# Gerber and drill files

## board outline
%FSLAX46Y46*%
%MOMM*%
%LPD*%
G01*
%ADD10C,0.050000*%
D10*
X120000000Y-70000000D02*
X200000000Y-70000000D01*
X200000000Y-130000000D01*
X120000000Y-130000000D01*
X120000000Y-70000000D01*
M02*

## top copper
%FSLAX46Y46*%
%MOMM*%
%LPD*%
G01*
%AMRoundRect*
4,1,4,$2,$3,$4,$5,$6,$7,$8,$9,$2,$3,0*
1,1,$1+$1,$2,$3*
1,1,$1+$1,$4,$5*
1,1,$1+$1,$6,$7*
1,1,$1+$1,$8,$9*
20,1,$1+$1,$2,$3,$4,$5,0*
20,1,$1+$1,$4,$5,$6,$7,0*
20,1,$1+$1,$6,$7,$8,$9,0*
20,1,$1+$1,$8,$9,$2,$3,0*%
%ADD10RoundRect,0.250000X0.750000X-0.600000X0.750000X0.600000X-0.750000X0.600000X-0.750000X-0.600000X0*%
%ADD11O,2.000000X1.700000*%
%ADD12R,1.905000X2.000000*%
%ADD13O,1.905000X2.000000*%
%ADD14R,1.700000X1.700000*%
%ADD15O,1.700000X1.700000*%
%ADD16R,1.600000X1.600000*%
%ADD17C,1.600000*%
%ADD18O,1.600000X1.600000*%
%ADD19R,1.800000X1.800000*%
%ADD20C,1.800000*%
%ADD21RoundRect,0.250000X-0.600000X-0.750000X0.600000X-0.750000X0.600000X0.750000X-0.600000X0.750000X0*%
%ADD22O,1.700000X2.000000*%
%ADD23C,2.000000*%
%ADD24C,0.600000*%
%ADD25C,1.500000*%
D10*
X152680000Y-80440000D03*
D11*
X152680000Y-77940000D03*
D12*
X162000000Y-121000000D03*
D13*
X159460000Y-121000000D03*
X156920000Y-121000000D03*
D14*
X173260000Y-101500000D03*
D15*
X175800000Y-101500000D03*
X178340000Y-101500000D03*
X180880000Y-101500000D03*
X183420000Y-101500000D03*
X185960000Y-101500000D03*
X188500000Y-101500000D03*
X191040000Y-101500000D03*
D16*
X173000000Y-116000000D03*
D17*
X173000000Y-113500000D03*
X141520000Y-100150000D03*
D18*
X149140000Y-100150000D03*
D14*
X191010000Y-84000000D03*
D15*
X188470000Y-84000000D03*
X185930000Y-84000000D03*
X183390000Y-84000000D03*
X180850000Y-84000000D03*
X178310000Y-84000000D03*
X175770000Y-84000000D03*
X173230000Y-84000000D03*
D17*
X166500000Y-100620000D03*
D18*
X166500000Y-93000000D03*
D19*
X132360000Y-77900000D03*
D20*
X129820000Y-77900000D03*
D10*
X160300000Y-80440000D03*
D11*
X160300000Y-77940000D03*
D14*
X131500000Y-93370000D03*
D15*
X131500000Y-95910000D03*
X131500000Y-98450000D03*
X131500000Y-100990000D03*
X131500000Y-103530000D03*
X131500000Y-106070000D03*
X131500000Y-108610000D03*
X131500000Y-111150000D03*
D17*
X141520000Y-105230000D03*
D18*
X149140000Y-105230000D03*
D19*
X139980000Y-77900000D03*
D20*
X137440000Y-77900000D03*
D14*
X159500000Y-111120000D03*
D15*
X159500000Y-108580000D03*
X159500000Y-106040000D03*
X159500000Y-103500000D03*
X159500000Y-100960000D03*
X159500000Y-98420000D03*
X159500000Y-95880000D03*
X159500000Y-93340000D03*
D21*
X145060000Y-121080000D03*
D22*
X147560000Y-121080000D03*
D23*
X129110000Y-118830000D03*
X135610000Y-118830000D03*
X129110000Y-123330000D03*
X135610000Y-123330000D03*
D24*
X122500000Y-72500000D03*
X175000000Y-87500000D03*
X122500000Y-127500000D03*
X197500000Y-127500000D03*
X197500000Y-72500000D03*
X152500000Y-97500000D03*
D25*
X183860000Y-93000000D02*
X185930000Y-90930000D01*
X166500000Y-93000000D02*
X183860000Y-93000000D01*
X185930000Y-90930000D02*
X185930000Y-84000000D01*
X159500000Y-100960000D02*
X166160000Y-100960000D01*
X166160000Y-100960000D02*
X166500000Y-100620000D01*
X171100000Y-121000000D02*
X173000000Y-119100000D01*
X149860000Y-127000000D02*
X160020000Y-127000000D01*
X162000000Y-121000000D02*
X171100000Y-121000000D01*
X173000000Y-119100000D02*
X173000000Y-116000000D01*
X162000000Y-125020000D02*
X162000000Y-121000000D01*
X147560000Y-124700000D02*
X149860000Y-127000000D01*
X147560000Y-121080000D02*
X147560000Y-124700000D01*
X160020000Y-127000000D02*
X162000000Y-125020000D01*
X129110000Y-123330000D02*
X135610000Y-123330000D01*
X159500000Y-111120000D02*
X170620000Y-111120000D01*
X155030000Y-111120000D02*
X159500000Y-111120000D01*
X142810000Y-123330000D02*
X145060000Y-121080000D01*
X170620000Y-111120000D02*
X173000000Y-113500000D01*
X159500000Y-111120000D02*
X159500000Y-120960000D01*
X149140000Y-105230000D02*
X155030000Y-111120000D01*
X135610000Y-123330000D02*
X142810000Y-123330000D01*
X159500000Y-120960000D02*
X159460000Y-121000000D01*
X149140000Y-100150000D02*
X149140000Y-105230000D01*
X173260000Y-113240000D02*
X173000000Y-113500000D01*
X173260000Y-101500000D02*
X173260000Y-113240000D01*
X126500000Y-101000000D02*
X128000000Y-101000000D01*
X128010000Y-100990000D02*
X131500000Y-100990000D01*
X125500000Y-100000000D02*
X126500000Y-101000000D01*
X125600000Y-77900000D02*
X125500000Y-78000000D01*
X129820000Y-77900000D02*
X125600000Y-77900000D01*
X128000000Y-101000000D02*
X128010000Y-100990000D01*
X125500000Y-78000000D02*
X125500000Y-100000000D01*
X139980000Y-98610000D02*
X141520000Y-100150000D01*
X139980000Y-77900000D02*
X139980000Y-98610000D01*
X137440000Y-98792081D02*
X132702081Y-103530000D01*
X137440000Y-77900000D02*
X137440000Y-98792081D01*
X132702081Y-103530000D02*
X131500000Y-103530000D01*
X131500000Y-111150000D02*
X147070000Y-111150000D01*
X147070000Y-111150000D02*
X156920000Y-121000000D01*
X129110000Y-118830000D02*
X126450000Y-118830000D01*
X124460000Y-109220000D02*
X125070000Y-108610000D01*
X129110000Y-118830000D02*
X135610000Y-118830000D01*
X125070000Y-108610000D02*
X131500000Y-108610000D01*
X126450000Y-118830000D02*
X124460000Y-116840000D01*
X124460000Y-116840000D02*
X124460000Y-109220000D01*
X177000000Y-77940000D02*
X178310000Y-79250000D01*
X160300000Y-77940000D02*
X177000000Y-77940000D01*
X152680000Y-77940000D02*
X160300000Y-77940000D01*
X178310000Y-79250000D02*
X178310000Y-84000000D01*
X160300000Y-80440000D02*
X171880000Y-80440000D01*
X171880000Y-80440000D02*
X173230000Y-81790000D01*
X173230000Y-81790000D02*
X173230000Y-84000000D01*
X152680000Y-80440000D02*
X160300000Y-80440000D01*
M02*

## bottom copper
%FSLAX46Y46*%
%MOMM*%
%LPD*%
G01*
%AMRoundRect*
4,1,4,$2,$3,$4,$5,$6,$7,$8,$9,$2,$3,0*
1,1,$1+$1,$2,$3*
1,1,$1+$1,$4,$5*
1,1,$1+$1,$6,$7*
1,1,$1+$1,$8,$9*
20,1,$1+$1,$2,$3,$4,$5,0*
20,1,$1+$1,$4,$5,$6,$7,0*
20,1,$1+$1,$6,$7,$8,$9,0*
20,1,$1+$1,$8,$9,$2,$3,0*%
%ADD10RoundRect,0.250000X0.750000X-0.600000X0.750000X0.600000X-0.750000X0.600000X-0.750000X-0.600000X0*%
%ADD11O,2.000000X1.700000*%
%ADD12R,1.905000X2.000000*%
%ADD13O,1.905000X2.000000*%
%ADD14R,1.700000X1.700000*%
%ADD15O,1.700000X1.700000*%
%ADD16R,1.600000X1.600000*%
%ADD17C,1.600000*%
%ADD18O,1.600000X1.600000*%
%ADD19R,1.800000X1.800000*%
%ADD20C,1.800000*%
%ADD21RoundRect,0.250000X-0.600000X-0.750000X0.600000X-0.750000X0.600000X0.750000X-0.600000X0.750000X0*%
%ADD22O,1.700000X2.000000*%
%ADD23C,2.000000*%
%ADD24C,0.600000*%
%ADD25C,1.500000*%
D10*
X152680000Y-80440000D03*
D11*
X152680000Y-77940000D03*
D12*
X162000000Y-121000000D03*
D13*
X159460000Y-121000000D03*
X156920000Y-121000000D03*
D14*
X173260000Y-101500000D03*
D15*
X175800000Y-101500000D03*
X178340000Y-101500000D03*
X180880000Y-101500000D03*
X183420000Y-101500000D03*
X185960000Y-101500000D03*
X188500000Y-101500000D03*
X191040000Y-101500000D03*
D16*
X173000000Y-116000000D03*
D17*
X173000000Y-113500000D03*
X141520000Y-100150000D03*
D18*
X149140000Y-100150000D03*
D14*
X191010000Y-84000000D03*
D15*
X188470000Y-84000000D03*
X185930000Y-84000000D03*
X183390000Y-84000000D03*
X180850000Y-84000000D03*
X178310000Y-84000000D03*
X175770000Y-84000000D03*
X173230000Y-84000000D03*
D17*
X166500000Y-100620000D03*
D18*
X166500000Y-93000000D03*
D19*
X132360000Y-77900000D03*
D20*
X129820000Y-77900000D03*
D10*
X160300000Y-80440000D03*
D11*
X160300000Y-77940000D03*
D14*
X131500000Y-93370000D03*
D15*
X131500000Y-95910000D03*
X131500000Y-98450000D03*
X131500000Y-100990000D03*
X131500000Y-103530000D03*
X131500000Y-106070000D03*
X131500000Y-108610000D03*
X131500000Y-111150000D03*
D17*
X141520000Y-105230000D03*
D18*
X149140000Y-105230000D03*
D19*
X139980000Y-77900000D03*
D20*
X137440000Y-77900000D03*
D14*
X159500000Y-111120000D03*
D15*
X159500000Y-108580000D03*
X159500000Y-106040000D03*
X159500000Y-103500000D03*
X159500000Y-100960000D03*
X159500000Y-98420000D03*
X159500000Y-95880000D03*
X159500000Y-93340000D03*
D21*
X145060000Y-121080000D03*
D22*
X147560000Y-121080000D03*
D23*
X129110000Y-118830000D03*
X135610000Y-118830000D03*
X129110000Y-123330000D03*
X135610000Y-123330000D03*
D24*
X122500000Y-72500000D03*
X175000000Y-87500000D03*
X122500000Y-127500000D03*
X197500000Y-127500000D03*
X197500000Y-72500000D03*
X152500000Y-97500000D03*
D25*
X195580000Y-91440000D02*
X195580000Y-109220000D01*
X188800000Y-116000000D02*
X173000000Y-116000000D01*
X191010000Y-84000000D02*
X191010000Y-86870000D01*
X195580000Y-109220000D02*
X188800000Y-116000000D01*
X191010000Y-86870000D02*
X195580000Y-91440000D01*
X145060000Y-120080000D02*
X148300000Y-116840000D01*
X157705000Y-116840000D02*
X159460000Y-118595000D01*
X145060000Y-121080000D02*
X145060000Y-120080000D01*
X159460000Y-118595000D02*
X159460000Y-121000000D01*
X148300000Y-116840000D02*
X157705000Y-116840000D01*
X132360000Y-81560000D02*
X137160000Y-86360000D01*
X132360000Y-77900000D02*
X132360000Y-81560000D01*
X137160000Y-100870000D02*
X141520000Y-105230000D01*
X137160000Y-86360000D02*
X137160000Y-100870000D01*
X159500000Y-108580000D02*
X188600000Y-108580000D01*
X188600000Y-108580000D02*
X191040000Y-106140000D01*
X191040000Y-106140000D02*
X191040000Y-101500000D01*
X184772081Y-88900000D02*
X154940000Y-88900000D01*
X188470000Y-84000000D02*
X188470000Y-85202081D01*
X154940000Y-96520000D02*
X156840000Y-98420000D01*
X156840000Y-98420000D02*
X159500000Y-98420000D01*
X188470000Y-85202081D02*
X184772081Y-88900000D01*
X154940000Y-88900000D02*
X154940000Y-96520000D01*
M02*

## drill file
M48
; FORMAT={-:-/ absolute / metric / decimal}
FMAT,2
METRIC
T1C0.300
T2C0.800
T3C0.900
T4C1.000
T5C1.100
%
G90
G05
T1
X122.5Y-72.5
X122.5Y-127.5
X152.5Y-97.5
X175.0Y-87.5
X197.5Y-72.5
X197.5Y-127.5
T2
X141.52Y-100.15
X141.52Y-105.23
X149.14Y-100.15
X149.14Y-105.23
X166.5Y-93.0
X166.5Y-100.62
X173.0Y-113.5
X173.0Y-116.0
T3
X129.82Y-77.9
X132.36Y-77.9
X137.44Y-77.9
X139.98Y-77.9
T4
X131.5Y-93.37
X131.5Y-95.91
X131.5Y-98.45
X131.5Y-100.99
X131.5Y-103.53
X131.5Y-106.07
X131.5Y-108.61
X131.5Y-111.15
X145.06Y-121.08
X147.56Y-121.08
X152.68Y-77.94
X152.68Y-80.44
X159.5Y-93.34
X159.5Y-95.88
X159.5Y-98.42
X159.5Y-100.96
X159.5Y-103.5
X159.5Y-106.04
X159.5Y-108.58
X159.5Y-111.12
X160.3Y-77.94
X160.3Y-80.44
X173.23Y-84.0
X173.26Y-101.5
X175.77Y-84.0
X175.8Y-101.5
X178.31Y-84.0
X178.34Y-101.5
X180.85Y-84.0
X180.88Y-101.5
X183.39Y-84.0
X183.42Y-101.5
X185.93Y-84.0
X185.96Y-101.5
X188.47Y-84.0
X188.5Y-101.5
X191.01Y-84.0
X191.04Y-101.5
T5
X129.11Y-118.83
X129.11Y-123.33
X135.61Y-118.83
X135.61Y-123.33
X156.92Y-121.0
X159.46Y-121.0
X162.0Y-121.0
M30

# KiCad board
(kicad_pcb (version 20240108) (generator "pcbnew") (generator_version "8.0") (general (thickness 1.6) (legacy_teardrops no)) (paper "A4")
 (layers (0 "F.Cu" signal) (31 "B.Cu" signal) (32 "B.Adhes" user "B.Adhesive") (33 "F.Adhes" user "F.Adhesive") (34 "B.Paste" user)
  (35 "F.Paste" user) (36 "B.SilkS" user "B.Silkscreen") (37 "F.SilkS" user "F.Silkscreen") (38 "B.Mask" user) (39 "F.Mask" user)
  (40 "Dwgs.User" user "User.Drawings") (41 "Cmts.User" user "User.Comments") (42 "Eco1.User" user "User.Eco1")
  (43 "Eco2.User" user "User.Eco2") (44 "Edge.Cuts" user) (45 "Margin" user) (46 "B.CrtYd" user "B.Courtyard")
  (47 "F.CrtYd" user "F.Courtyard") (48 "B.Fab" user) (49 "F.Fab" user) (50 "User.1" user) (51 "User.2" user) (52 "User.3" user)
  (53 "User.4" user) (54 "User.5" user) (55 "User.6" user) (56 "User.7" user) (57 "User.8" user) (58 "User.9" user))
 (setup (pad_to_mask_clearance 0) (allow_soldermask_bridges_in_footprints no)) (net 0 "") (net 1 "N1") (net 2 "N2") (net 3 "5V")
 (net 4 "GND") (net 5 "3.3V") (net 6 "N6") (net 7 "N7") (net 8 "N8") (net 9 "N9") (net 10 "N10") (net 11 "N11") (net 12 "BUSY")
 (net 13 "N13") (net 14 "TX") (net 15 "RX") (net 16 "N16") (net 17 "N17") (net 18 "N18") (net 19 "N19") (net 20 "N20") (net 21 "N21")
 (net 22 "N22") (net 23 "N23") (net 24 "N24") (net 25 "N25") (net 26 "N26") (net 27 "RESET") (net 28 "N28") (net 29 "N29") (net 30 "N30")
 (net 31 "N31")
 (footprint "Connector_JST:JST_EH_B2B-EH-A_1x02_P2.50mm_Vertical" (layer "F.Cu") (at 152.68 80.44 90)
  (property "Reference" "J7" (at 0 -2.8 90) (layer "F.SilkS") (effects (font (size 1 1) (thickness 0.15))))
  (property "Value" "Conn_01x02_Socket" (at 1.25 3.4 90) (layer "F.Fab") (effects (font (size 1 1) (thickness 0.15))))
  (pad "1" thru_hole roundrect (at 0 0 90) (size 1.7 2) (drill 1) (layers "*.Cu" "*.Mask") (remove_unused_layers no)
   (roundrect_rratio 0.147059) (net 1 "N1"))
  (pad "2" thru_hole oval (at 2.5 0 90) (size 1.7 2) (drill 1) (layers "*.Cu" "*.Mask") (remove_unused_layers no) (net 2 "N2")))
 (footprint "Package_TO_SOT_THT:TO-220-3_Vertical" (layer "F.Cu") (at 162 121 180)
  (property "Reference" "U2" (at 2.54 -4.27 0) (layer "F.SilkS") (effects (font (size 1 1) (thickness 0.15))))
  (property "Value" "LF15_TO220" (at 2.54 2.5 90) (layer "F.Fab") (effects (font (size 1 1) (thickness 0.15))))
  (pad "1" thru_hole rect (at 0 0 180) (size 1.905 2) (drill 1.1) (layers "*.Cu" "*.Mask") (remove_unused_layers no) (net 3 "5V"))
  (pad "2" thru_hole oval (at 2.54 0 180) (size 1.905 2) (drill 1.1) (layers "*.Cu" "*.Mask") (remove_unused_layers no) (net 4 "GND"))
  (pad "3" thru_hole oval (at 5.08 0 180) (size 1.905 2) (drill 1.1) (layers "*.Cu" "*.Mask") (remove_unused_layers no) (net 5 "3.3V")))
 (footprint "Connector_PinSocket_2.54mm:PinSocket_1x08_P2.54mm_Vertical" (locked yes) (layer "F.Cu") (at 173.26 101.5 90)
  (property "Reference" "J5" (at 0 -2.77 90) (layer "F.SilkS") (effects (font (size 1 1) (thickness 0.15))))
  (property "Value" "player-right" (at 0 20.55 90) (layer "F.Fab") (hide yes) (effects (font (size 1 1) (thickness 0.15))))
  (pad "1" thru_hole rect (at 0 0 90) (size 1.7 1.7) (drill 1) (layers "*.Cu" "*.Mask") (remove_unused_layers no) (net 4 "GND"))
  (pad "2" thru_hole oval (at 0 2.54 90) (size 1.7 1.7) (drill 1) (layers "*.Cu" "*.Mask") (remove_unused_layers no) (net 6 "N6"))
  (pad "3" thru_hole oval (at 0 5.08 90) (size 1.7 1.7) (drill 1) (layers "*.Cu" "*.Mask") (remove_unused_layers no) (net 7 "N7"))
  (pad "4" thru_hole oval (at 0 7.62 90) (size 1.7 1.7) (drill 1) (layers "*.Cu" "*.Mask") (remove_unused_layers no) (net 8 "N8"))
  (pad "5" thru_hole oval (at 0 10.16 90) (size 1.7 1.7) (drill 1) (layers "*.Cu" "*.Mask") (remove_unused_layers no) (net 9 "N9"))
  (pad "6" thru_hole oval (at 0 12.7 90) (size 1.7 1.7) (drill 1) (layers "*.Cu" "*.Mask") (remove_unused_layers no) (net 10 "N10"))
  (pad "7" thru_hole oval (at 0 15.24 90) (size 1.7 1.7) (drill 1) (layers "*.Cu" "*.Mask") (remove_unused_layers no) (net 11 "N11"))
  (pad "8" thru_hole oval (at 0 17.78 90) (size 1.7 1.7) (drill 1) (layers "*.Cu" "*.Mask") (remove_unused_layers no) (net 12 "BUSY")))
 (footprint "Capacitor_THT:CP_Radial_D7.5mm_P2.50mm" (layer "F.Cu") (at 173 116 90)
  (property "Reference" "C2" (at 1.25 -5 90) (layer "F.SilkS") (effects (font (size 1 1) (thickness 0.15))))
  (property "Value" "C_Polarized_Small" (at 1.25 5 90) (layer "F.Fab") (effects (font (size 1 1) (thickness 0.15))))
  (pad "1" thru_hole rect (at 0 0 90) (size 1.6 1.6) (drill 0.8) (layers "*.Cu" "*.Mask") (remove_unused_layers no) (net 3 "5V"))
  (pad "2" thru_hole circle (at 2.5 0 90) (size 1.6 1.6) (drill 0.8) (layers "*.Cu" "*.Mask") (remove_unused_layers no) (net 4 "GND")))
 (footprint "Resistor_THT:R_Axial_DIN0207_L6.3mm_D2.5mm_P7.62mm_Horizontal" (layer "F.Cu") (at 141.52 100.15)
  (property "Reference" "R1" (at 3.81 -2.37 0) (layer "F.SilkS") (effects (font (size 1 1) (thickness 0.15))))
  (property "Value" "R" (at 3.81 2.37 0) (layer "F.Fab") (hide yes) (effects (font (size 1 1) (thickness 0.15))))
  (pad "1" thru_hole circle (at 0 0) (size 1.6 1.6) (drill 0.8) (layers "*.Cu" "*.Mask") (remove_unused_layers no) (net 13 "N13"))
  (pad "2" thru_hole oval (at 7.62 0) (size 1.6 1.6) (drill 0.8) (layers "*.Cu" "*.Mask") (remove_unused_layers no) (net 4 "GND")))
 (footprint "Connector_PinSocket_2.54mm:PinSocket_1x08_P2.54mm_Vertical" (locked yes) (layer "F.Cu") (at 191.01 84 -90)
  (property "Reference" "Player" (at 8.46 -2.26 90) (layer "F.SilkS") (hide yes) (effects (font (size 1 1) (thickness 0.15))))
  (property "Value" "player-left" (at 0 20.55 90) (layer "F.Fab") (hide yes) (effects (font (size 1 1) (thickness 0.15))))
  (pad "1" thru_hole rect (at 0 0 270) (size 1.7 1.7) (drill 1) (layers "*.Cu" "*.Mask") (remove_unused_layers no) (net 3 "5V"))
  (pad "2" thru_hole oval (at 0 2.54 270) (size 1.7 1.7) (drill 1) (layers "*.Cu" "*.Mask") (remove_unused_layers no) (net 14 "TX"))
  (pad "3" thru_hole oval (at 0 5.08 270) (size 1.7 1.7) (drill 1) (layers "*.Cu" "*.Mask") (remove_unused_layers no) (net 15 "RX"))
  (pad "4" thru_hole oval (at 0 7.62 270) (size 1.7 1.7) (drill 1) (layers "*.Cu" "*.Mask") (remove_unused_layers no) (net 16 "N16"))
  (pad "5" thru_hole oval (at 0 10.16 270) (size 1.7 1.7) (drill 1) (layers "*.Cu" "*.Mask") (remove_unused_layers no) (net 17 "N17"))
  (pad "6" thru_hole oval (at 0 12.7 270) (size 1.7 1.7) (drill 1) (layers "*.Cu" "*.Mask") (remove_unused_layers no) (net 2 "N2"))
  (pad "7" thru_hole oval (at 0 15.24 270) (size 1.7 1.7) (drill 1) (layers "*.Cu" "*.Mask") (remove_unused_layers no) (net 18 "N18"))
  (pad "8" thru_hole oval (at 0 17.78 270) (size 1.7 1.7) (drill 1) (layers "*.Cu" "*.Mask") (remove_unused_layers no) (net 1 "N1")))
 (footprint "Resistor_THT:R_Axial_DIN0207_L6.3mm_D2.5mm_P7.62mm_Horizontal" (layer "F.Cu") (at 166.5 100.62 90)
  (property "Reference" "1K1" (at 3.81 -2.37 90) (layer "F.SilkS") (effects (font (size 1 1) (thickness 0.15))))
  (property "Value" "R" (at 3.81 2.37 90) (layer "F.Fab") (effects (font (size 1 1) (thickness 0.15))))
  (pad "1" thru_hole circle (at 0 0 90) (size 1.6 1.6) (drill 0.8) (layers "*.Cu" "*.Mask") (remove_unused_layers no) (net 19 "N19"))
  (pad "2" thru_hole oval (at 7.62 0 90) (size 1.6 1.6) (drill 0.8) (layers "*.Cu" "*.Mask") (remove_unused_layers no) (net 15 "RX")))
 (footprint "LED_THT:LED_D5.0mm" (layer "F.Cu") (at 132.36 77.9 180)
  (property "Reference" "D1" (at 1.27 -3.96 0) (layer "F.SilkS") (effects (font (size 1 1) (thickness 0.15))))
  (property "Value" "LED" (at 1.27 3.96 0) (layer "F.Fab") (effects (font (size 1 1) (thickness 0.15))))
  (pad "1" thru_hole rect (at 0 0 180) (size 1.8 1.8) (drill 0.9) (layers "*.Cu" "*.Mask") (remove_unused_layers no) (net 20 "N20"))
  (pad "2" thru_hole circle (at 2.54 0 180) (size 1.8 1.8) (drill 0.9) (layers "*.Cu" "*.Mask") (remove_unused_layers no) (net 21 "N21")))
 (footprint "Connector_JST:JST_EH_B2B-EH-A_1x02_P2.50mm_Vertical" (layer "F.Cu") (at 160.3 80.44 90)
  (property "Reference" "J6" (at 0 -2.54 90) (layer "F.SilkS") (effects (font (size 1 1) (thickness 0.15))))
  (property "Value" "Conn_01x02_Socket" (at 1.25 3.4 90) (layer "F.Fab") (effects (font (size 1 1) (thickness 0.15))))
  (pad "1" thru_hole roundrect (at 0 0 90) (size 1.7 2) (drill 1) (layers "*.Cu" "*.Mask") (remove_unused_layers no)
   (roundrect_rratio 0.147059) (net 1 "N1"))
  (pad "2" thru_hole oval (at 2.5 0 90) (size 1.7 2) (drill 1) (layers "*.Cu" "*.Mask") (remove_unused_layers no) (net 2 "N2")))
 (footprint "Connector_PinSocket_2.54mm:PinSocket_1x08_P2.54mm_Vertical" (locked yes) (layer "F.Cu") (at 131.5 93.37)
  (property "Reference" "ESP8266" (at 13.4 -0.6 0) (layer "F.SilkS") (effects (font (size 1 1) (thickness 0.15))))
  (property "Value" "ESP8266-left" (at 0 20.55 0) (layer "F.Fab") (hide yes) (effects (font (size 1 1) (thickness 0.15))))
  (pad "1" thru_hole rect (at 0 0) (size 1.7 1.7) (drill 1) (layers "*.Cu" "*.Mask") (remove_unused_layers no) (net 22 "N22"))
  (pad "2" thru_hole oval (at 0 2.54) (size 1.7 1.7) (drill 1) (layers "*.Cu" "*.Mask") (remove_unused_layers no) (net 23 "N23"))
  (pad "3" thru_hole oval (at 0 5.08) (size 1.7 1.7) (drill 1) (layers "*.Cu" "*.Mask") (remove_unused_layers no) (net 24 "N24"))
  (pad "4" thru_hole oval (at 0 7.62) (size 1.7 1.7) (drill 1) (layers "*.Cu" "*.Mask") (remove_unused_layers no) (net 21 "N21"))
  (pad "5" thru_hole oval (at 0 10.16) (size 1.7 1.7) (drill 1) (layers "*.Cu" "*.Mask") (remove_unused_layers no) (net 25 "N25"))
  (pad "6" thru_hole oval (at 0 12.7) (size 1.7 1.7) (drill 1) (layers "*.Cu" "*.Mask") (remove_unused_layers no) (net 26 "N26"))
  (pad "7" thru_hole oval (at 0 15.24) (size 1.7 1.7) (drill 1) (layers "*.Cu" "*.Mask") (remove_unused_layers no) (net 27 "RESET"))
  (pad "8" thru_hole oval (at 0 17.78) (size 1.7 1.7) (drill 1) (layers "*.Cu" "*.Mask") (remove_unused_layers no) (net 5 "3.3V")))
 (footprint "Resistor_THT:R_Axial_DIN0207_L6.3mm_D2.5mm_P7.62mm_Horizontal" (layer "F.Cu") (at 141.52 105.23)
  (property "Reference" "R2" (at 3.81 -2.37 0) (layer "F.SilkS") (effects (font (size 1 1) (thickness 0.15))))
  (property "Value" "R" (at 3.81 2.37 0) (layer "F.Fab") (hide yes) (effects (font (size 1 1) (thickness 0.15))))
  (pad "1" thru_hole circle (at 0 0) (size 1.6 1.6) (drill 0.8) (layers "*.Cu" "*.Mask") (remove_unused_layers no) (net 20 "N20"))
  (pad "2" thru_hole oval (at 7.62 0) (size 1.6 1.6) (drill 0.8) (layers "*.Cu" "*.Mask") (remove_unused_layers no) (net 4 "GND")))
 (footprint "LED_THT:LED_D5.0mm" (layer "F.Cu") (at 139.98 77.9 180)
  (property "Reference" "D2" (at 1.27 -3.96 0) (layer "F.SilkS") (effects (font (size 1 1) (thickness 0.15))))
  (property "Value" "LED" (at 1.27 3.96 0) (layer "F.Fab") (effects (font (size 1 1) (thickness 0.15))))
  (pad "1" thru_hole rect (at 0 0 180) (size 1.8 1.8) (drill 0.9) (layers "*.Cu" "*.Mask") (remove_unused_layers no) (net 13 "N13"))
  (pad "2" thru_hole circle (at 2.54 0 180) (size 1.8 1.8) (drill 0.9) (layers "*.Cu" "*.Mask") (remove_unused_layers no) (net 25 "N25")))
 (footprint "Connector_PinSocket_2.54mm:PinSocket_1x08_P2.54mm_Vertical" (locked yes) (layer "F.Cu") (at 159.5 111.12 180)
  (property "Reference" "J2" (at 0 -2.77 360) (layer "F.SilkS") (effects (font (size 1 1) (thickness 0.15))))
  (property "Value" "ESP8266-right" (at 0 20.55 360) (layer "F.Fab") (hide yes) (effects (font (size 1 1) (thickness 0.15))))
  (pad "1" thru_hole rect (at 0 0 180) (size 1.7 1.7) (drill 1) (layers "*.Cu" "*.Mask") (remove_unused_layers no) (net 4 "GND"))
  (pad "2" thru_hole oval (at 0 2.54 180) (size 1.7 1.7) (drill 1) (layers "*.Cu" "*.Mask") (remove_unused_layers no) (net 12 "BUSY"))
  (pad "3" thru_hole oval (at 0 5.08 180) (size 1.7 1.7) (drill 1) (layers "*.Cu" "*.Mask") (remove_unused_layers no) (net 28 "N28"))
  (pad "4" thru_hole oval (at 0 7.62 180) (size 1.7 1.7) (drill 1) (layers "*.Cu" "*.Mask") (remove_unused_layers no) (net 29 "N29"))
  (pad "5" thru_hole oval (at 0 10.16 180) (size 1.7 1.7) (drill 1) (layers "*.Cu" "*.Mask") (remove_unused_layers no) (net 19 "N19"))
  (pad "6" thru_hole oval (at 0 12.7 180) (size 1.7 1.7) (drill 1) (layers "*.Cu" "*.Mask") (remove_unused_layers no) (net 14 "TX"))
  (pad "7" thru_hole oval (at 0 15.24 180) (size 1.7 1.7) (drill 1) (layers "*.Cu" "*.Mask") (remove_unused_layers no) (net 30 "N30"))
  (pad "8" thru_hole oval (at 0 17.78 180) (size 1.7 1.7) (drill 1) (layers "*.Cu" "*.Mask") (remove_unused_layers no) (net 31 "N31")))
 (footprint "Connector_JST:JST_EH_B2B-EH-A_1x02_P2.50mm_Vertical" (layer "F.Cu") (at 145.06 121.08)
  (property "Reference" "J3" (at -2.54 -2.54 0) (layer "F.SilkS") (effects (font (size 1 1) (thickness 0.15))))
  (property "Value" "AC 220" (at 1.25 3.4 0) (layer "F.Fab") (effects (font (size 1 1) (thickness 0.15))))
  (pad "1" thru_hole roundrect (at 0 0) (size 1.7 2) (drill 1) (layers "*.Cu" "*.Mask") (remove_unused_layers no)
   (roundrect_rratio 0.147059) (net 4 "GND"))
  (pad "2" thru_hole oval (at 2.5 0) (size 1.7 2) (drill 1) (layers "*.Cu" "*.Mask") (remove_unused_layers no) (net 3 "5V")))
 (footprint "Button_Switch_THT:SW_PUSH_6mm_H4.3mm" (layer "F.Cu") (at 129.11 118.83)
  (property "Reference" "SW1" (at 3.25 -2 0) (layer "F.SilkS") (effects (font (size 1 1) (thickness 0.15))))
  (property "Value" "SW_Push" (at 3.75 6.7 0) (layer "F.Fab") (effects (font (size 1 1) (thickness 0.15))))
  (pad "1" thru_hole circle (at 0 0 90) (size 2 2) (drill 1.1) (layers "*.Cu" "*.Mask") (remove_unused_layers no) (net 27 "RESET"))
  (pad "1" thru_hole circle (at 6.5 0 90) (size 2 2) (drill 1.1) (layers "*.Cu" "*.Mask") (remove_unused_layers no) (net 27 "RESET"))
  (pad "2" thru_hole circle (at 0 4.5 90) (size 2 2) (drill 1.1) (layers "*.Cu" "*.Mask") (remove_unused_layers no) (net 4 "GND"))
  (pad "2" thru_hole circle (at 6.5 4.5 90) (size 2 2) (drill 1.1) (layers "*.Cu" "*.Mask") (remove_unused_layers no) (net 4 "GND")))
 (gr_rect (start 120 70) (end 200 130) (stroke (width 0.05) (type default)) (fill none) (layer "Edge.Cuts"))
 (via (at 122.5 72.5) (size 0.6) (drill 0.3) (layers "F.Cu" "B.Cu") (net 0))
 (via (at 175 87.5) (size 0.6) (drill 0.3) (layers "F.Cu" "B.Cu") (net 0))
 (via (at 122.5 127.5) (size 0.6) (drill 0.3) (layers "F.Cu" "B.Cu") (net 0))
 (via (at 197.5 127.5) (size 0.6) (drill 0.3) (layers "F.Cu" "B.Cu") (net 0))
 (via (at 197.5 72.5) (size 0.6) (drill 0.3) (layers "F.Cu" "B.Cu") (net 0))
 (via (at 152.5 97.5) (size 0.6) (drill 0.3) (layers "F.Cu" "B.Cu") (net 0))
 (segment (start 183.86 93) (end 185.93 90.93) (width 1.5) (layer "F.Cu") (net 15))
 (segment (start 166.5 93) (end 183.86 93) (width 1.5) (layer "F.Cu") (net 15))
 (segment (start 185.93 90.93) (end 185.93 84) (width 1.5) (layer "F.Cu") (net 15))
 (segment (start 159.5 100.96) (end 166.16 100.96) (width 1.5) (layer "F.Cu") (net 19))
 (segment (start 166.16 100.96) (end 166.5 100.62) (width 1.5) (layer "F.Cu") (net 19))
 (segment (start 171.1 121) (end 173 119.1) (width 1.5) (layer "F.Cu") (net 3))
 (segment (start 149.86 127) (end 160.02 127) (width 1.5) (layer "F.Cu") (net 3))
 (segment (start 162 121) (end 171.1 121) (width 1.5) (layer "F.Cu") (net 3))
 (segment (start 173 119.1) (end 173 116) (width 1.5) (layer "F.Cu") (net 3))
 (segment (start 162 125.02) (end 162 121) (width 1.5) (layer "F.Cu") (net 3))
 (segment (start 147.56 124.7) (end 149.86 127) (width 1.5) (layer "F.Cu") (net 3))
 (segment (start 147.56 121.08) (end 147.56 124.7) (width 1.5) (layer "F.Cu") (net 3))
 (segment (start 160.02 127) (end 162 125.02) (width 1.5) (layer "F.Cu") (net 3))
 (segment (start 195.58 91.44) (end 195.58 109.22) (width 1.5) (layer "B.Cu") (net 3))
 (segment (start 188.8 116) (end 173 116) (width 1.5) (layer "B.Cu") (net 3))
 (segment (start 191.01 84) (end 191.01 86.87) (width 1.5) (layer "B.Cu") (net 3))
 (segment (start 195.58 109.22) (end 188.8 116) (width 1.5) (layer "B.Cu") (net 3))
 (segment (start 191.01 86.87) (end 195.58 91.44) (width 1.5) (layer "B.Cu") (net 3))
 (segment (start 129.11 123.33) (end 135.61 123.33) (width 1.5) (layer "F.Cu") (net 4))
 (segment (start 159.5 111.12) (end 170.62 111.12) (width 1.5) (layer "F.Cu") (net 4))
 (segment (start 155.03 111.12) (end 159.5 111.12) (width 1.5) (layer "F.Cu") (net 4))
 (segment (start 142.81 123.33) (end 145.06 121.08) (width 1.5) (layer "F.Cu") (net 4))
 (segment (start 170.62 111.12) (end 173 113.5) (width 1.5) (layer "F.Cu") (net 4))
 (segment (start 159.5 111.12) (end 159.5 120.96) (width 1.5) (layer "F.Cu") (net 4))
 (segment (start 149.14 105.23) (end 155.03 111.12) (width 1.5) (layer "F.Cu") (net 4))
 (segment (start 135.61 123.33) (end 142.81 123.33) (width 1.5) (layer "F.Cu") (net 4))
 (segment (start 159.5 120.96) (end 159.46 121) (width 1.5) (layer "F.Cu") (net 4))
 (segment (start 149.14 100.15) (end 149.14 105.23) (width 1.5) (layer "F.Cu") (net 4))
 (segment (start 173.26 113.24) (end 173 113.5) (width 1.5) (layer "F.Cu") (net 4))
 (segment (start 173.26 101.5) (end 173.26 113.24) (width 1.5) (layer "F.Cu") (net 4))
 (segment (start 145.06 120.08) (end 148.3 116.84) (width 1.5) (layer "B.Cu") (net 4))
 (segment (start 157.705 116.84) (end 159.46 118.595) (width 1.5) (layer "B.Cu") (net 4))
 (segment (start 145.06 121.08) (end 145.06 120.08) (width 1.5) (layer "B.Cu") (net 4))
 (segment (start 159.46 118.595) (end 159.46 121) (width 1.5) (layer "B.Cu") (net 4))
 (segment (start 148.3 116.84) (end 157.705 116.84) (width 1.5) (layer "B.Cu") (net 4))
 (segment (start 132.36 81.56) (end 137.16 86.36) (width 1.5) (layer "B.Cu") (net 20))
 (segment (start 132.36 77.9) (end 132.36 81.56) (width 1.5) (layer "B.Cu") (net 20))
 (segment (start 137.16 100.87) (end 141.52 105.23) (width 1.5) (layer "B.Cu") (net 20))
 (segment (start 137.16 86.36) (end 137.16 100.87) (width 1.5) (layer "B.Cu") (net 20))
 (segment (start 126.5 101) (end 128 101) (width 1.5) (layer "F.Cu") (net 21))
 (segment (start 128.01 100.99) (end 131.5 100.99) (width 1.5) (layer "F.Cu") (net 21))
 (segment (start 125.5 100) (end 126.5 101) (width 1.5) (layer "F.Cu") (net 21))
 (segment (start 125.6 77.9) (end 125.5 78) (width 1.5) (layer "F.Cu") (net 21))
 (segment (start 129.82 77.9) (end 125.6 77.9) (width 1.5) (layer "F.Cu") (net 21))
 (segment (start 128 101) (end 128.01 100.99) (width 1.5) (layer "F.Cu") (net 21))
 (segment (start 125.5 78) (end 125.5 100) (width 1.5) (layer "F.Cu") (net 21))
 (segment (start 139.98 98.61) (end 141.52 100.15) (width 1.5) (layer "F.Cu") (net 13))
 (segment (start 139.98 77.9) (end 139.98 98.61) (width 1.5) (layer "F.Cu") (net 13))
 (segment (start 137.44 98.792081) (end 132.702081 103.53) (width 1.5) (layer "F.Cu") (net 25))
 (segment (start 137.44 77.9) (end 137.44 98.792081) (width 1.5) (layer "F.Cu") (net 25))
 (segment (start 132.702081 103.53) (end 131.5 103.53) (width 1.5) (layer "F.Cu") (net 25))
 (segment (start 131.5 111.15) (end 147.07 111.15) (width 1.5) (layer "F.Cu") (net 5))
 (segment (start 147.07 111.15) (end 156.92 121) (width 1.5) (layer "F.Cu") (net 5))
 (segment (start 129.11 118.83) (end 126.45 118.83) (width 1.5) (layer "F.Cu") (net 27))
 (segment (start 124.46 109.22) (end 125.07 108.61) (width 1.5) (layer "F.Cu") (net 27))
 (segment (start 129.11 118.83) (end 135.61 118.83) (width 1.5) (layer "F.Cu") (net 27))
 (segment (start 125.07 108.61) (end 131.5 108.61) (width 1.5) (layer "F.Cu") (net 27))
 (segment (start 126.45 118.83) (end 124.46 116.84) (width 1.5) (layer "F.Cu") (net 27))
 (segment (start 124.46 116.84) (end 124.46 109.22) (width 1.5) (layer "F.Cu") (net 27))
 (segment (start 159.5 108.58) (end 188.6 108.58) (width 1.5) (layer "B.Cu") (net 12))
 (segment (start 188.6 108.58) (end 191.04 106.14) (width 1.5) (layer "B.Cu") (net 12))
 (segment (start 191.04 106.14) (end 191.04 101.5) (width 1.5) (layer "B.Cu") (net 12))
 (segment (start 184.772081 88.9) (end 154.94 88.9) (width 1.5) (layer "B.Cu") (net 14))
 (segment (start 188.47 84) (end 188.47 85.202081) (width 1.5) (layer "B.Cu") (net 14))
 (segment (start 154.94 96.52) (end 156.84 98.42) (width 1.5) (layer "B.Cu") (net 14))
 (segment (start 156.84 98.42) (end 159.5 98.42) (width 1.5) (layer "B.Cu") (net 14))
 (segment (start 188.47 85.202081) (end 184.772081 88.9) (width 1.5) (layer "B.Cu") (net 14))
 (segment (start 154.94 88.9) (end 154.94 96.52) (width 1.5) (layer "B.Cu") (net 14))
 (segment (start 177 77.94) (end 178.31 79.25) (width 1.5) (layer "F.Cu") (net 2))
 (segment (start 160.3 77.94) (end 177 77.94) (width 1.5) (layer "F.Cu") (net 2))
 (segment (start 152.68 77.94) (end 160.3 77.94) (width 1.5) (layer "F.Cu") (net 2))
 (segment (start 178.31 79.25) (end 178.31 84) (width 1.5) (layer "F.Cu") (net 2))
 (segment (start 160.3 80.44) (end 171.88 80.44) (width 1.5) (layer "F.Cu") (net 1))
 (segment (start 171.88 80.44) (end 173.23 81.79) (width 1.5) (layer "F.Cu") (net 1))
 (segment (start 173.23 81.79) (end 173.23 84) (width 1.5) (layer "F.Cu") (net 1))
 (segment (start 152.68 80.44) (end 160.3 80.44) (width 1.5) (layer "F.Cu") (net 1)))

